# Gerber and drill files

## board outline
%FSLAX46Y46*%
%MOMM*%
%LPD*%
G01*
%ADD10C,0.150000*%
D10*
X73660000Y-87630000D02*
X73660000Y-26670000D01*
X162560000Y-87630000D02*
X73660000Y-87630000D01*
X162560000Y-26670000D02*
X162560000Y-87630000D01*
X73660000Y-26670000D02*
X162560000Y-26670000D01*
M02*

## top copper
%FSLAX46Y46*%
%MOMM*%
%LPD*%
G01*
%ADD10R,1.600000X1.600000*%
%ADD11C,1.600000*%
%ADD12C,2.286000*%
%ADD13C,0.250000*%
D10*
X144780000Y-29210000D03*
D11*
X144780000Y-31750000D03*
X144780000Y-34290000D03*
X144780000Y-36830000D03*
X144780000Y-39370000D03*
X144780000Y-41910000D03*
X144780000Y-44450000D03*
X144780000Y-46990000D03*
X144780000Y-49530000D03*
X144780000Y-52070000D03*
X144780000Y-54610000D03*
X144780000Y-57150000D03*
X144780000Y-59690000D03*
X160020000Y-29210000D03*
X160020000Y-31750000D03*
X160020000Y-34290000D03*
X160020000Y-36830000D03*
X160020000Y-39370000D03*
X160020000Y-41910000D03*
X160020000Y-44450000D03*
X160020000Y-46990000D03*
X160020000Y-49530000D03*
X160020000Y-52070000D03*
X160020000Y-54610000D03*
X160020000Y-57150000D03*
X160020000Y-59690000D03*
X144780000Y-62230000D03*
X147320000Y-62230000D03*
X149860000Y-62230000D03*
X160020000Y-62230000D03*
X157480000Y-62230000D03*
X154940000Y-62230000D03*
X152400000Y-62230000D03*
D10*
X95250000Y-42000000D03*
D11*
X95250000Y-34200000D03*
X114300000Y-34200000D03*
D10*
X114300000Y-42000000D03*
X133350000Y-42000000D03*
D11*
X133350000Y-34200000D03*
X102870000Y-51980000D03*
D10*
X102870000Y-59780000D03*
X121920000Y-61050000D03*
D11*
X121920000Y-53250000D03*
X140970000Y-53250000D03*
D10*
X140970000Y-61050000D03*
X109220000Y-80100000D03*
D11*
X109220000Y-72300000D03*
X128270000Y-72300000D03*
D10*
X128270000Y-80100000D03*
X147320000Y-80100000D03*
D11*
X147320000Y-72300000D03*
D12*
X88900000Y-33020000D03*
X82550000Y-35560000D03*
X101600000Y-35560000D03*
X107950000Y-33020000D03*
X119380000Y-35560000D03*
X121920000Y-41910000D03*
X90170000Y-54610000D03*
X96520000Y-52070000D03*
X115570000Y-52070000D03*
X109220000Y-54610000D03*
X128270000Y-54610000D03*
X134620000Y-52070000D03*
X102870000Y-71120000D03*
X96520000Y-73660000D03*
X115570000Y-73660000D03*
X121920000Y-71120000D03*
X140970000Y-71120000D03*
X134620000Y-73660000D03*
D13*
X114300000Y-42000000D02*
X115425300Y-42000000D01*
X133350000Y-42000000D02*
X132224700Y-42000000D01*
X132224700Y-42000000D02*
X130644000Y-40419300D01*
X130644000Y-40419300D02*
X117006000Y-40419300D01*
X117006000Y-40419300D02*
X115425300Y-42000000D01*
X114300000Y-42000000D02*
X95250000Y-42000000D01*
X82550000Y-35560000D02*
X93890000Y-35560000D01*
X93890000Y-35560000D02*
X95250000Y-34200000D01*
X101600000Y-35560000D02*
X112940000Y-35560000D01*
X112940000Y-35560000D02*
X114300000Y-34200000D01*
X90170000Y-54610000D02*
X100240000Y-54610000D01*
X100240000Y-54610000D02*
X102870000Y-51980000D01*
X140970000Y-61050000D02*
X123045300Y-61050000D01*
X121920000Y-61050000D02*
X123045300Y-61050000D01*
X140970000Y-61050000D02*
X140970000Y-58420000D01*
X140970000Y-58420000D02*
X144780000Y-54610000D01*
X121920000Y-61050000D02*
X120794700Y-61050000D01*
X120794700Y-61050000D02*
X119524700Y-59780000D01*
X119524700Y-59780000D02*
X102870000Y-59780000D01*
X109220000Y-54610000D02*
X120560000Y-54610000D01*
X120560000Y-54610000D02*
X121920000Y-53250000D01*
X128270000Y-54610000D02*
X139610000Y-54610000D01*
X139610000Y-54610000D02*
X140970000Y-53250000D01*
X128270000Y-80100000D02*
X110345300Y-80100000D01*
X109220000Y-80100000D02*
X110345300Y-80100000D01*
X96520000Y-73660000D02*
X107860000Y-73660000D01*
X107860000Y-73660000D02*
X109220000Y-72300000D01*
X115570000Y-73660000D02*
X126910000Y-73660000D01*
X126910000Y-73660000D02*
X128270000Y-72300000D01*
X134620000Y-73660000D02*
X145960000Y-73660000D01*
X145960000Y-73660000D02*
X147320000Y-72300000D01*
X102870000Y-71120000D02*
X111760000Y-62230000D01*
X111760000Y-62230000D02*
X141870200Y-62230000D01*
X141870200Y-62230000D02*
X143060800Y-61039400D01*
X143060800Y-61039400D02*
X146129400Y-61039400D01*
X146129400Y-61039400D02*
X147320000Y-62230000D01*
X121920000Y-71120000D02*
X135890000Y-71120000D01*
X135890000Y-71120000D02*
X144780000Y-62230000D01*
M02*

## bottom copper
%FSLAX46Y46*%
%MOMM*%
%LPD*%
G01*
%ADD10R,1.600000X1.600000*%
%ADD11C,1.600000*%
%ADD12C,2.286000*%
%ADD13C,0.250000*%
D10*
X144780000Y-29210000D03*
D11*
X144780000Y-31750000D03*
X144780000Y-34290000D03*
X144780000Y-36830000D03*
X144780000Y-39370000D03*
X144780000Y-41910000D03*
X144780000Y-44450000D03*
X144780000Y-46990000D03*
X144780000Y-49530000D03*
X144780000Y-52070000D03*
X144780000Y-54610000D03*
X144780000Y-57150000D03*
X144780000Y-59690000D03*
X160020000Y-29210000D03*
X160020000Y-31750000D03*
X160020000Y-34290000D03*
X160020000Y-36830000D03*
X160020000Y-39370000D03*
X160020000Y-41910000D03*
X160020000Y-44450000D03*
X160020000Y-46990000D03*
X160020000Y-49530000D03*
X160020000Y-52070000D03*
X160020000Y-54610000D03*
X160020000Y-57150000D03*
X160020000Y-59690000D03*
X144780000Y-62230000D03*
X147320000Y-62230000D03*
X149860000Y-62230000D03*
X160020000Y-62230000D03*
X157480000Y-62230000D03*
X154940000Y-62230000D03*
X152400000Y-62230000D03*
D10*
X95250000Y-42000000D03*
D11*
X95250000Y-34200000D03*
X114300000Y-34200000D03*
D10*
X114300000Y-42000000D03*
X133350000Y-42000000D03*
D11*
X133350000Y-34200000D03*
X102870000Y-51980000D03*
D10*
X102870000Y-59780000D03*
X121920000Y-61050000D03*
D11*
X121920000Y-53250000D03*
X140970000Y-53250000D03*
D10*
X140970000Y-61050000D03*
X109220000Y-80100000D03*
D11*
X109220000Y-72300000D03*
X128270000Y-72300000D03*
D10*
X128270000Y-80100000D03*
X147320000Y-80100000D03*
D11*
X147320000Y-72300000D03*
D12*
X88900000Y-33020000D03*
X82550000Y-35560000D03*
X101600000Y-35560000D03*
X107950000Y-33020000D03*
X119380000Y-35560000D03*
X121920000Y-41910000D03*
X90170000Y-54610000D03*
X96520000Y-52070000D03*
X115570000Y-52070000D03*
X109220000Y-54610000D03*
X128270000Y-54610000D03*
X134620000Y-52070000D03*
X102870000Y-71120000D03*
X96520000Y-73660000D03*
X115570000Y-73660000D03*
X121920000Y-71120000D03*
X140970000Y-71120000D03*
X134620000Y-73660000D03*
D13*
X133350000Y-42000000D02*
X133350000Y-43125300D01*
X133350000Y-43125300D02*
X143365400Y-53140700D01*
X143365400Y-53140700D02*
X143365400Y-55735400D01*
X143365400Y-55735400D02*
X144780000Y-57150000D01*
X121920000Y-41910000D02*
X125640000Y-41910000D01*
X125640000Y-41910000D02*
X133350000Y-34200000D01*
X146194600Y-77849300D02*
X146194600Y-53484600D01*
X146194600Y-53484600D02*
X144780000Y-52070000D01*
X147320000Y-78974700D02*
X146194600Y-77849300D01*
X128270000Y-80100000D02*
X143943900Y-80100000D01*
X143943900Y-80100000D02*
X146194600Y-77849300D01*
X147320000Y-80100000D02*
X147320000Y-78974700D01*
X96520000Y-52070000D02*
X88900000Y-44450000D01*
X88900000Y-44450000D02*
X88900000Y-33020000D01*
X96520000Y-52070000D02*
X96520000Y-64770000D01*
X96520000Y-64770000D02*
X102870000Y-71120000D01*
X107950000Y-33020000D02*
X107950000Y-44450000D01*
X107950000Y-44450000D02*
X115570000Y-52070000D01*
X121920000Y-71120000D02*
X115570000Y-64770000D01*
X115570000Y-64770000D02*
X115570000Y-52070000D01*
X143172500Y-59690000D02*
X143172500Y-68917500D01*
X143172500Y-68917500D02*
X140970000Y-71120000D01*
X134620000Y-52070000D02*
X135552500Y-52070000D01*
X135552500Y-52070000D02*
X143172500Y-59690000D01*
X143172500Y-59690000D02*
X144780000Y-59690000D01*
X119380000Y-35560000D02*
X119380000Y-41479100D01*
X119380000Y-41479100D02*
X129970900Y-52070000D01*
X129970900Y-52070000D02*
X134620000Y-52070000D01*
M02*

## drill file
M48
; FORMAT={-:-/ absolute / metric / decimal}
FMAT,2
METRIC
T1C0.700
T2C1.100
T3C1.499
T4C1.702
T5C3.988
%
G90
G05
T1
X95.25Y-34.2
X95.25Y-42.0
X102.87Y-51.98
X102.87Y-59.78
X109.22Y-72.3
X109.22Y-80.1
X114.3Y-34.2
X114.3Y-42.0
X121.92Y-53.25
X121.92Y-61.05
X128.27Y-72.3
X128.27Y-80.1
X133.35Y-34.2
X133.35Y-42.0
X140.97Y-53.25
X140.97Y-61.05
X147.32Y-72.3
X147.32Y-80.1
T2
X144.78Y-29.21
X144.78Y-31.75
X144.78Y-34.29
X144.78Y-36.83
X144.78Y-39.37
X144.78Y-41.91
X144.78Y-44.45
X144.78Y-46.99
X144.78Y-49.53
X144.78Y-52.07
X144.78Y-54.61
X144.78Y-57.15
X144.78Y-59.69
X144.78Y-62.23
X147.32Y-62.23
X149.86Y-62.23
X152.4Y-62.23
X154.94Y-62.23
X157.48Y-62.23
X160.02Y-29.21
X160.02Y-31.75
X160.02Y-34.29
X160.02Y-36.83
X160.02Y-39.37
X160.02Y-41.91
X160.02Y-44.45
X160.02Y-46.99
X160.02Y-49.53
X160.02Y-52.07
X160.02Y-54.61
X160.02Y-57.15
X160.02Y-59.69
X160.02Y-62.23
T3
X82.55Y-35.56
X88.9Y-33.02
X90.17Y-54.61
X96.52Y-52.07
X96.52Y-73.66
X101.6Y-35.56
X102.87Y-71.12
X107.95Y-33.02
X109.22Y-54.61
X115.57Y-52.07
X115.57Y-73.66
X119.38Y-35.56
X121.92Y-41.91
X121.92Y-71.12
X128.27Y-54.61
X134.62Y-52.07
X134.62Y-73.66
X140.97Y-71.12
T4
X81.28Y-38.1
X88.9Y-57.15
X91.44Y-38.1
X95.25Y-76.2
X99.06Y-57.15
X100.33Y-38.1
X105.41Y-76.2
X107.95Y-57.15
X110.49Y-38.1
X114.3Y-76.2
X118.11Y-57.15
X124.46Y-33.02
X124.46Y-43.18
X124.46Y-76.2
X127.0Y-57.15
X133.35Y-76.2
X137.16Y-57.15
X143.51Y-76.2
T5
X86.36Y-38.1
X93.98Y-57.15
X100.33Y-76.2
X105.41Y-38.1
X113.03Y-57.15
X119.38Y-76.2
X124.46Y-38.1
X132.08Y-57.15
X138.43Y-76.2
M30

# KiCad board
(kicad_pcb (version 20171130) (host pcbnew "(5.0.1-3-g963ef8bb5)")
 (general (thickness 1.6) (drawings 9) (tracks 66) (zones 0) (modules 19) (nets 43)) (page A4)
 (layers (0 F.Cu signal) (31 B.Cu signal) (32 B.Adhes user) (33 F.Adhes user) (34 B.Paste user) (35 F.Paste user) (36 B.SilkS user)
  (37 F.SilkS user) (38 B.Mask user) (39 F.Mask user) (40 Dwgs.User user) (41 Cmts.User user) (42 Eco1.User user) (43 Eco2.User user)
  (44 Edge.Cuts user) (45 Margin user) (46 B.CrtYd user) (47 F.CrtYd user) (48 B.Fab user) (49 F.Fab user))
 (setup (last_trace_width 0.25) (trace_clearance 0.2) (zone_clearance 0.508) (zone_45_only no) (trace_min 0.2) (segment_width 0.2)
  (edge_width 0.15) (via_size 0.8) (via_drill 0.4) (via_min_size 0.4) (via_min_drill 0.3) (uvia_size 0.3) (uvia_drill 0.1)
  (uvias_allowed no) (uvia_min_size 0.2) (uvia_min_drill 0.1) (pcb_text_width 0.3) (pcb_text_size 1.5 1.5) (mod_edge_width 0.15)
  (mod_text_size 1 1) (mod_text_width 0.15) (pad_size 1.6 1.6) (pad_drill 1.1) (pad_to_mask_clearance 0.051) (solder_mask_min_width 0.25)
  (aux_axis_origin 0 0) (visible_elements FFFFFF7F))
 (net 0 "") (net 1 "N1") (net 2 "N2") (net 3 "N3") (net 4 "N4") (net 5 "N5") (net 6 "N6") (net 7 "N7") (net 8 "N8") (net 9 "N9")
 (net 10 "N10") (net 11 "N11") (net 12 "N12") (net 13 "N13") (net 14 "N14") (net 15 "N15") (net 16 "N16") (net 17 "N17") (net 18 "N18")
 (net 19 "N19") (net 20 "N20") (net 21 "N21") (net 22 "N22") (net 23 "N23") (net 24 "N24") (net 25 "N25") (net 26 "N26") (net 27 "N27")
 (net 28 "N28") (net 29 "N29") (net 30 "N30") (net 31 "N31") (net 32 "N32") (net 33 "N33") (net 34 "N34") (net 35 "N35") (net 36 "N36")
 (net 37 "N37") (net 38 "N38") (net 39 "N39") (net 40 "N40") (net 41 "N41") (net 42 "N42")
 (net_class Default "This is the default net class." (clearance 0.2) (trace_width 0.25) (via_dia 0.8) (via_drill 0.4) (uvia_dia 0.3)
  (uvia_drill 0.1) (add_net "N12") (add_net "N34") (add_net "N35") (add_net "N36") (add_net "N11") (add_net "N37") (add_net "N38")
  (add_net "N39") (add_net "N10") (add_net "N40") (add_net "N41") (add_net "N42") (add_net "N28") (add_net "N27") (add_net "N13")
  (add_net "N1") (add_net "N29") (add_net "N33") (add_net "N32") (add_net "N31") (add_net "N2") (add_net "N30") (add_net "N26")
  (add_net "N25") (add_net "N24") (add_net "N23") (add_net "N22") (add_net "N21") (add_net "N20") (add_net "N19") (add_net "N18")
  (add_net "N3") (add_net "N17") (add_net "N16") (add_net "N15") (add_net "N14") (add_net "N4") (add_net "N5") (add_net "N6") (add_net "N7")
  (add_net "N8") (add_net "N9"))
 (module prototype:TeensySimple (layer F.Cu) (at 152.4 45.72 270)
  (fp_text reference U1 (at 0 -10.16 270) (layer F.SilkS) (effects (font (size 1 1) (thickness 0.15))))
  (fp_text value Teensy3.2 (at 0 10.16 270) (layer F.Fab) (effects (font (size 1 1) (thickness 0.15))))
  (pad 1 thru_hole rect (at -16.51 7.62 270) (size 1.6 1.6) (drill 1.1) (layers *.Cu *.Mask F.SilkS) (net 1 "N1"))
  (pad 2 thru_hole circle (at -13.97 7.62 270) (size 1.6 1.6) (drill 1.1) (layers *.Cu *.Mask F.SilkS) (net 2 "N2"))
  (pad 3 thru_hole circle (at -11.43 7.62 270) (size 1.6 1.6) (drill 1.1) (layers *.Cu *.Mask F.SilkS) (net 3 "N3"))
  (pad 4 thru_hole circle (at -8.89 7.62 270) (size 1.6 1.6) (drill 1.1) (layers *.Cu *.Mask F.SilkS) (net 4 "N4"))
  (pad 5 thru_hole circle (at -6.35 7.62 270) (size 1.6 1.6) (drill 1.1) (layers *.Cu *.Mask F.SilkS) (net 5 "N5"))
  (pad 6 thru_hole circle (at -3.81 7.62 270) (size 1.6 1.6) (drill 1.1) (layers *.Cu *.Mask F.SilkS) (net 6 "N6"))
  (pad 7 thru_hole circle (at -1.27 7.62 270) (size 1.6 1.6) (drill 1.1) (layers *.Cu *.Mask F.SilkS) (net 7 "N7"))
  (pad 8 thru_hole circle (at 1.27 7.62 270) (size 1.6 1.6) (drill 1.1) (layers *.Cu *.Mask F.SilkS) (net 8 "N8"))
  (pad 9 thru_hole circle (at 3.81 7.62 270) (size 1.6 1.6) (drill 1.1) (layers *.Cu *.Mask F.SilkS) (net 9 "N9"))
  (pad 10 thru_hole circle (at 6.35 7.62 270) (size 1.6 1.6) (drill 1.1) (layers *.Cu *.Mask F.SilkS) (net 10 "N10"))
  (pad 11 thru_hole circle (at 8.89 7.62 270) (size 1.6 1.6) (drill 1.1) (layers *.Cu *.Mask F.SilkS) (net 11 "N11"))
  (pad 12 thru_hole circle (at 11.43 7.62 270) (size 1.6 1.6) (drill 1.1) (layers *.Cu *.Mask F.SilkS) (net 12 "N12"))
  (pad 13 thru_hole circle (at 13.97 7.62 270) (size 1.6 1.6) (drill 1.1) (layers *.Cu *.Mask F.SilkS) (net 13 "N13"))
  (pad 33 thru_hole circle (at -16.51 -7.62 270) (size 1.6 1.6) (drill 1.1) (layers *.Cu *.Mask F.SilkS) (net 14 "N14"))
  (pad 32 thru_hole circle (at -13.97 -7.62 270) (size 1.6 1.6) (drill 1.1) (layers *.Cu *.Mask F.SilkS) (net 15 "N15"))
  (pad 31 thru_hole circle (at -11.43 -7.62 270) (size 1.6 1.6) (drill 1.1) (layers *.Cu *.Mask F.SilkS) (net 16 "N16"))
  (pad 30 thru_hole circle (at -8.89 -7.62 270) (size 1.6 1.6) (drill 1.1) (layers *.Cu *.Mask F.SilkS) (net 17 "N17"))
  (pad 29 thru_hole circle (at -6.35 -7.62 270) (size 1.6 1.6) (drill 1.1) (layers *.Cu *.Mask F.SilkS) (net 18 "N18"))
  (pad 28 thru_hole circle (at -3.81 -7.62 270) (size 1.6 1.6) (drill 1.1) (layers *.Cu *.Mask F.SilkS) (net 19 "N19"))
  (pad 27 thru_hole circle (at -1.27 -7.62 270) (size 1.6 1.6) (drill 1.1) (layers *.Cu *.Mask F.SilkS) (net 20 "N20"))
  (pad 26 thru_hole circle (at 1.27 -7.62 270) (size 1.6 1.6) (drill 1.1) (layers *.Cu *.Mask F.SilkS) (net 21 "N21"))
  (pad 25 thru_hole circle (at 3.81 -7.62 270) (size 1.6 1.6) (drill 1.1) (layers *.Cu *.Mask F.SilkS) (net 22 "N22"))
  (pad 24 thru_hole circle (at 6.35 -7.62 270) (size 1.6 1.6) (drill 1.1) (layers *.Cu *.Mask F.SilkS) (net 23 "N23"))
  (pad 23 thru_hole circle (at 8.89 -7.62 270) (size 1.6 1.6) (drill 1.1) (layers *.Cu *.Mask F.SilkS) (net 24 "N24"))
  (pad 22 thru_hole circle (at 11.43 -7.62 270) (size 1.6 1.6) (drill 1.1) (layers *.Cu *.Mask F.SilkS) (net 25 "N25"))
  (pad 21 thru_hole circle (at 13.97 -7.62 270) (size 1.6 1.6) (drill 1.1) (layers *.Cu *.Mask F.SilkS) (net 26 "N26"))
  (pad 14 thru_hole circle (at 16.51 7.62 270) (size 1.6 1.6) (drill 1.1) (layers *.Cu *.Mask F.SilkS) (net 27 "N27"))
  (pad 15 thru_hole circle (at 16.51 5.08 270) (size 1.6 1.6) (drill 1.1) (layers *.Cu *.Mask F.SilkS) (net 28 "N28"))
  (pad 16 thru_hole circle (at 16.51 2.54 270) (size 1.6 1.6) (drill 1.1) (layers *.Cu *.Mask F.SilkS) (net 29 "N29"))
  (pad 20 thru_hole circle (at 16.51 -7.62 270) (size 1.6 1.6) (drill 1.1) (layers *.Cu *.Mask F.SilkS) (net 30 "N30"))
  (pad 19 thru_hole circle (at 16.51 -5.08 270) (size 1.6 1.6) (drill 1.1) (layers *.Cu *.Mask F.SilkS) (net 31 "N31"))
  (pad 18 thru_hole circle (at 16.51 -2.54 270) (size 1.6 1.6) (drill 1.1) (layers *.Cu *.Mask F.SilkS) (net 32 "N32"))
  (pad 17 thru_hole circle (at 16.51 0 270) (size 1.6 1.6) (drill 1.1) (layers *.Cu *.Mask F.SilkS) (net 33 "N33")))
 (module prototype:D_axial (layer F.Cu) (at 95.25 38.1 90)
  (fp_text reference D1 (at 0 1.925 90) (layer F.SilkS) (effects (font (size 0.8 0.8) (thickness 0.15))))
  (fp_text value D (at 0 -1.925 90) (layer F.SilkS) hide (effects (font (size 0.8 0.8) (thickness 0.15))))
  (pad 1 thru_hole rect (at -3.9 0 90) (size 1.6 1.6) (drill 0.7) (layers *.Cu *.Mask F.SilkS) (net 12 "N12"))
  (pad 2 thru_hole circle (at 3.9 0 90) (size 1.6 1.6) (drill 0.7) (layers *.Cu *.Mask F.SilkS) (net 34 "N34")))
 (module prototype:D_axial (layer F.Cu) (at 114.3 38.1 90)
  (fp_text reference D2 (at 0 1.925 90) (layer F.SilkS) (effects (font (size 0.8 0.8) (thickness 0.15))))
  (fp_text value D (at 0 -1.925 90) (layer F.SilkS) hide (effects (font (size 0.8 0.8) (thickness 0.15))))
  (pad 2 thru_hole circle (at 3.9 0 90) (size 1.6 1.6) (drill 0.7) (layers *.Cu *.Mask F.SilkS) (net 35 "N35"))
  (pad 1 thru_hole rect (at -3.9 0 90) (size 1.6 1.6) (drill 0.7) (layers *.Cu *.Mask F.SilkS) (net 12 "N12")))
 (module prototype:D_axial (layer F.Cu) (at 133.35 38.1 90)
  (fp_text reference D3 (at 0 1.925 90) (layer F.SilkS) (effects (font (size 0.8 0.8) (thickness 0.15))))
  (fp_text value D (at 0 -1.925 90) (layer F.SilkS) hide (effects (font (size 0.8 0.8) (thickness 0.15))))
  (pad 1 thru_hole rect (at -3.9 0 90) (size 1.6 1.6) (drill 0.7) (layers *.Cu *.Mask F.SilkS) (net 12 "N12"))
  (pad 2 thru_hole circle (at 3.9 0 90) (size 1.6 1.6) (drill 0.7) (layers *.Cu *.Mask F.SilkS) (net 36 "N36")))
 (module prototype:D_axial (layer F.Cu) (at 102.87 55.88 90)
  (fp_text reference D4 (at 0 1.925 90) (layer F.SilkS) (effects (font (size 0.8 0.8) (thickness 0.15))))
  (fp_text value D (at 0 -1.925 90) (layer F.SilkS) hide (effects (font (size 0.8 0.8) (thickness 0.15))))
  (pad 2 thru_hole circle (at 3.9 0 90) (size 1.6 1.6) (drill 0.7) (layers *.Cu *.Mask F.SilkS) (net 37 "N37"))
  (pad 1 thru_hole rect (at -3.9 0 90) (size 1.6 1.6) (drill 0.7) (layers *.Cu *.Mask F.SilkS) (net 11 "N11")))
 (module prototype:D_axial (layer F.Cu) (at 121.92 57.15 90)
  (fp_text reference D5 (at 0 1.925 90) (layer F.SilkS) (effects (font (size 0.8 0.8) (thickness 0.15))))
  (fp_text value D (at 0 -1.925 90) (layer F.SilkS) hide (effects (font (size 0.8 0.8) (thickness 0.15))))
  (pad 1 thru_hole rect (at -3.9 0 90) (size 1.6 1.6) (drill 0.7) (layers *.Cu *.Mask F.SilkS) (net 11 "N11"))
  (pad 2 thru_hole circle (at 3.9 0 90) (size 1.6 1.6) (drill 0.7) (layers *.Cu *.Mask F.SilkS) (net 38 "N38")))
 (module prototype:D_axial (layer F.Cu) (at 140.97 57.15 90)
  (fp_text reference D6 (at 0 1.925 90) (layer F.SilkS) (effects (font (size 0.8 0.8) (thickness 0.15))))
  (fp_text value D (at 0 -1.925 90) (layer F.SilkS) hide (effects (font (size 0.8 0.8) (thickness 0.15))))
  (pad 2 thru_hole circle (at 3.9 0 90) (size 1.6 1.6) (drill 0.7) (layers *.Cu *.Mask F.SilkS) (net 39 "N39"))
  (pad 1 thru_hole rect (at -3.9 0 90) (size 1.6 1.6) (drill 0.7) (layers *.Cu *.Mask F.SilkS) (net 11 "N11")))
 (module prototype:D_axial (layer F.Cu) (at 109.22 76.2 90)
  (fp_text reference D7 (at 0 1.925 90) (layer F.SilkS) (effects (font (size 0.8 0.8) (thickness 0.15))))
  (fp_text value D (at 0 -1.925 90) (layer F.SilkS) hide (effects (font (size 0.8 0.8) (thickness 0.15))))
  (pad 1 thru_hole rect (at -3.9 0 90) (size 1.6 1.6) (drill 0.7) (layers *.Cu *.Mask F.SilkS) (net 10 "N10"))
  (pad 2 thru_hole circle (at 3.9 0 90) (size 1.6 1.6) (drill 0.7) (layers *.Cu *.Mask F.SilkS) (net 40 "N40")))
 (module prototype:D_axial (layer F.Cu) (at 128.27 76.2 90)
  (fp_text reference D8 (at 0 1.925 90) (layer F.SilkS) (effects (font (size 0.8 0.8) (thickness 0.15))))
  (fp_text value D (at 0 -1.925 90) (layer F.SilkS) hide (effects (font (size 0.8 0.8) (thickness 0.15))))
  (pad 2 thru_hole circle (at 3.9 0 90) (size 1.6 1.6) (drill 0.7) (layers *.Cu *.Mask F.SilkS) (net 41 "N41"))
  (pad 1 thru_hole rect (at -3.9 0 90) (size 1.6 1.6) (drill 0.7) (layers *.Cu *.Mask F.SilkS) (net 10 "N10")))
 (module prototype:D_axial (layer F.Cu) (at 147.32 76.2 90)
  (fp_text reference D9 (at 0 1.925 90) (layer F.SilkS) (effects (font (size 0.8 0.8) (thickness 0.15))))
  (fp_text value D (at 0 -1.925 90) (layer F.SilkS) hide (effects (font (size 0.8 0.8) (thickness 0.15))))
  (pad 1 thru_hole rect (at -3.9 0 90) (size 1.6 1.6) (drill 0.7) (layers *.Cu *.Mask F.SilkS) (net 10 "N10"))
  (pad 2 thru_hole circle (at 3.9 0 90) (size 1.6 1.6) (drill 0.7) (layers *.Cu *.Mask F.SilkS) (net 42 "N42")))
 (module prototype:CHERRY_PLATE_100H (layer F.Cu) (at 86.36 38.1)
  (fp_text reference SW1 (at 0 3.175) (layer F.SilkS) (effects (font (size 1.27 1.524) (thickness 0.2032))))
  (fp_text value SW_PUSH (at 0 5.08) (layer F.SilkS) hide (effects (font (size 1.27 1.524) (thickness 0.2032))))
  (pad 1 thru_hole circle (at 2.54 -5.08) (size 2.286 2.286) (drill 1.4986) (layers *.Cu *.SilkS *.Mask) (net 28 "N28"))
  (pad 2 thru_hole circle (at -3.81 -2.54) (size 2.286 2.286) (drill 1.4986) (layers *.Cu *.SilkS *.Mask) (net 34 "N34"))
  (pad HOLE np_thru_hole circle (at 0 0) (size 3.9878 3.9878) (drill 3.9878) (layers *.Cu))
  (pad HOLE np_thru_hole circle (at -5.08 0) (size 1.7018 1.7018) (drill 1.7018) (layers *.Cu))
  (pad HOLE np_thru_hole circle (at 5.08 0) (size 1.7018 1.7018) (drill 1.7018) (layers *.Cu)))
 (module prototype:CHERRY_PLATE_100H (layer F.Cu) (at 105.41 38.1)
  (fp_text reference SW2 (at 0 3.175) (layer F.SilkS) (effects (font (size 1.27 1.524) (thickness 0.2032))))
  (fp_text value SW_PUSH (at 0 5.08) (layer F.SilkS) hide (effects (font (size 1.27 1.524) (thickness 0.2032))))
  (pad HOLE np_thru_hole circle (at 5.08 0) (size 1.7018 1.7018) (drill 1.7018) (layers *.Cu))
  (pad HOLE np_thru_hole circle (at -5.08 0) (size 1.7018 1.7018) (drill 1.7018) (layers *.Cu))
  (pad HOLE np_thru_hole circle (at 0 0) (size 3.9878 3.9878) (drill 3.9878) (layers *.Cu))
  (pad 2 thru_hole circle (at -3.81 -2.54) (size 2.286 2.286) (drill 1.4986) (layers *.Cu *.SilkS *.Mask) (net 35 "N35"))
  (pad 1 thru_hole circle (at 2.54 -5.08) (size 2.286 2.286) (drill 1.4986) (layers *.Cu *.SilkS *.Mask) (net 27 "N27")))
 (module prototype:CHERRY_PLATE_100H (layer F.Cu) (at 124.46 38.1 90)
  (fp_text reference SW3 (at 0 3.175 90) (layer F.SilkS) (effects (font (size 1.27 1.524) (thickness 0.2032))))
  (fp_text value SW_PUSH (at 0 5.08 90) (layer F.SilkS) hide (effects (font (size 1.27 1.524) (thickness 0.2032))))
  (pad 1 thru_hole circle (at 2.54 -5.08 90) (size 2.286 2.286) (drill 1.4986) (layers *.Cu *.SilkS *.Mask) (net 13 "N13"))
  (pad 2 thru_hole circle (at -3.81 -2.54 90) (size 2.286 2.286) (drill 1.4986) (layers *.Cu *.SilkS *.Mask) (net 36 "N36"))
  (pad HOLE np_thru_hole circle (at 0 0 90) (size 3.9878 3.9878) (drill 3.9878) (layers *.Cu))
  (pad HOLE np_thru_hole circle (at -5.08 0 90) (size 1.7018 1.7018) (drill 1.7018) (layers *.Cu))
  (pad HOLE np_thru_hole circle (at 5.08 0 90) (size 1.7018 1.7018) (drill 1.7018) (layers *.Cu)))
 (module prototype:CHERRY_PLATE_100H (layer F.Cu) (at 93.98 57.15)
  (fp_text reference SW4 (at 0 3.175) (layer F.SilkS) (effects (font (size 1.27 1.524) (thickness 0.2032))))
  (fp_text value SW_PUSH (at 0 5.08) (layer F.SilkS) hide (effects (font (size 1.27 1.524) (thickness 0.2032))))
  (pad HOLE np_thru_hole circle (at 5.08 0) (size 1.7018 1.7018) (drill 1.7018) (layers *.Cu))
  (pad HOLE np_thru_hole circle (at -5.08 0) (size 1.7018 1.7018) (drill 1.7018) (layers *.Cu))
  (pad HOLE np_thru_hole circle (at 0 0) (size 3.9878 3.9878) (drill 3.9878) (layers *.Cu))
  (pad 2 thru_hole circle (at -3.81 -2.54) (size 2.286 2.286) (drill 1.4986) (layers *.Cu *.SilkS *.Mask) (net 37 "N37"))
  (pad 1 thru_hole circle (at 2.54 -5.08) (size 2.286 2.286) (drill 1.4986) (layers *.Cu *.SilkS *.Mask) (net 28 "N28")))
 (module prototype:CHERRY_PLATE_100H (layer F.Cu) (at 113.03 57.15)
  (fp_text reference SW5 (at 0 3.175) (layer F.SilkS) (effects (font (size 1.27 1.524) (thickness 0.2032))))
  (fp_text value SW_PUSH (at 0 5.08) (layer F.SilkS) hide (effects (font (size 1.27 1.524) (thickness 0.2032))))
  (pad 1 thru_hole circle (at 2.54 -5.08) (size 2.286 2.286) (drill 1.4986) (layers *.Cu *.SilkS *.Mask) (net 27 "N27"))
  (pad 2 thru_hole circle (at -3.81 -2.54) (size 2.286 2.286) (drill 1.4986) (layers *.Cu *.SilkS *.Mask) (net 38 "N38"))
  (pad HOLE np_thru_hole circle (at 0 0) (size 3.9878 3.9878) (drill 3.9878) (layers *.Cu))
  (pad HOLE np_thru_hole circle (at -5.08 0) (size 1.7018 1.7018) (drill 1.7018) (layers *.Cu))
  (pad HOLE np_thru_hole circle (at 5.08 0) (size 1.7018 1.7018) (drill 1.7018) (layers *.Cu)))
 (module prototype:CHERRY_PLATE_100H (layer F.Cu) (at 132.08 57.15)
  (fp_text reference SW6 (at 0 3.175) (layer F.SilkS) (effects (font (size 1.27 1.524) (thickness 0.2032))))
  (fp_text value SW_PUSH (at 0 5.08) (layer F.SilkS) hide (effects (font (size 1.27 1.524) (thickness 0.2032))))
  (pad HOLE np_thru_hole circle (at 5.08 0) (size 1.7018 1.7018) (drill 1.7018) (layers *.Cu))
  (pad HOLE np_thru_hole circle (at -5.08 0) (size 1.7018 1.7018) (drill 1.7018) (layers *.Cu))
  (pad HOLE np_thru_hole circle (at 0 0) (size 3.9878 3.9878) (drill 3.9878) (layers *.Cu))
  (pad 2 thru_hole circle (at -3.81 -2.54) (size 2.286 2.286) (drill 1.4986) (layers *.Cu *.SilkS *.Mask) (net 39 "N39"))
  (pad 1 thru_hole circle (at 2.54 -5.08) (size 2.286 2.286) (drill 1.4986) (layers *.Cu *.SilkS *.Mask) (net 13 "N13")))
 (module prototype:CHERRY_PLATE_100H (layer F.Cu) (at 100.33 76.2)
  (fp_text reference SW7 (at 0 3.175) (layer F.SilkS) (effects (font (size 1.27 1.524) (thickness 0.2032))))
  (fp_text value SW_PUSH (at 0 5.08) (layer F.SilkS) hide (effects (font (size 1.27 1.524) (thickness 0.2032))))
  (pad 1 thru_hole circle (at 2.54 -5.08) (size 2.286 2.286) (drill 1.4986) (layers *.Cu *.SilkS *.Mask) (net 28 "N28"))
  (pad 2 thru_hole circle (at -3.81 -2.54) (size 2.286 2.286) (drill 1.4986) (layers *.Cu *.SilkS *.Mask) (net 40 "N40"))
  (pad HOLE np_thru_hole circle (at 0 0) (size 3.9878 3.9878) (drill 3.9878) (layers *.Cu))
  (pad HOLE np_thru_hole circle (at -5.08 0) (size 1.7018 1.7018) (drill 1.7018) (layers *.Cu))
  (pad HOLE np_thru_hole circle (at 5.08 0) (size 1.7018 1.7018) (drill 1.7018) (layers *.Cu)))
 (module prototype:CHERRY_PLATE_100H (layer F.Cu) (at 119.38 76.2)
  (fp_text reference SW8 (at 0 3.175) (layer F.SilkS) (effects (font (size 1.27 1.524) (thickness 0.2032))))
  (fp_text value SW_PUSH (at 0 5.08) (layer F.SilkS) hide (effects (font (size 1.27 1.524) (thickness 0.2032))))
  (pad HOLE np_thru_hole circle (at 5.08 0) (size 1.7018 1.7018) (drill 1.7018) (layers *.Cu))
  (pad HOLE np_thru_hole circle (at -5.08 0) (size 1.7018 1.7018) (drill 1.7018) (layers *.Cu))
  (pad HOLE np_thru_hole circle (at 0 0) (size 3.9878 3.9878) (drill 3.9878) (layers *.Cu))
  (pad 2 thru_hole circle (at -3.81 -2.54) (size 2.286 2.286) (drill 1.4986) (layers *.Cu *.SilkS *.Mask) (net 41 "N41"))
  (pad 1 thru_hole circle (at 2.54 -5.08) (size 2.286 2.286) (drill 1.4986) (layers *.Cu *.SilkS *.Mask) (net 27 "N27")))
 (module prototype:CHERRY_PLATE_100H (layer F.Cu) (at 138.43 76.2)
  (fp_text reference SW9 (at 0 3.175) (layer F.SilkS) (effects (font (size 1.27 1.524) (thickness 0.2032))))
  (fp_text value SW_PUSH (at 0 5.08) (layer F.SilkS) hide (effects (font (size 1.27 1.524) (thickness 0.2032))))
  (pad 1 thru_hole circle (at 2.54 -5.08) (size 2.286 2.286) (drill 1.4986) (layers *.Cu *.SilkS *.Mask) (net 13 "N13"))
  (pad 2 thru_hole circle (at -3.81 -2.54) (size 2.286 2.286) (drill 1.4986) (layers *.Cu *.SilkS *.Mask) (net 42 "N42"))
  (pad HOLE np_thru_hole circle (at 0 0) (size 3.9878 3.9878) (drill 3.9878) (layers *.Cu))
  (pad HOLE np_thru_hole circle (at -5.08 0) (size 1.7018 1.7018) (drill 1.7018) (layers *.Cu))
  (pad HOLE np_thru_hole circle (at 5.08 0) (size 1.7018 1.7018) (drill 1.7018) (layers *.Cu)))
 (gr_line (start 73.66 87.63) (end 73.66 26.67) (layer Edge.Cuts) (width 0.15))
 (gr_line (start 162.56 87.63) (end 73.66 87.63) (layer Edge.Cuts) (width 0.15))
 (gr_line (start 162.56 26.67) (end 162.56 87.63) (layer Edge.Cuts) (width 0.15))
 (gr_line (start 73.66 26.67) (end 162.56 26.67) (layer Edge.Cuts) (width 0.15))
 (segment (start 133.35 42) (end 133.35 43.1253) (width 0.25) (layer B.Cu) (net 12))
 (segment (start 133.35 43.1253) (end 143.3654 53.1407) (width 0.25) (layer B.Cu) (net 12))
 (segment (start 143.3654 53.1407) (end 143.3654 55.7354) (width 0.25) (layer B.Cu) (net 12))
 (segment (start 143.3654 55.7354) (end 144.78 57.15) (width 0.25) (layer B.Cu) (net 12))
 (segment (start 114.3 42) (end 115.4253 42) (width 0.25) (layer F.Cu) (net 12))
 (segment (start 133.35 42) (end 132.2247 42) (width 0.25) (layer F.Cu) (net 12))
 (segment (start 132.2247 42) (end 130.644 40.4193) (width 0.25) (layer F.Cu) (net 12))
 (segment (start 130.644 40.4193) (end 117.006 40.4193) (width 0.25) (layer F.Cu) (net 12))
 (segment (start 117.006 40.4193) (end 115.4253 42) (width 0.25) (layer F.Cu) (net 12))
 (segment (start 114.3 42) (end 95.25 42) (width 0.25) (layer F.Cu) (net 12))
 (segment (start 82.55 35.56) (end 93.89 35.56) (width 0.25) (layer F.Cu) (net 34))
 (segment (start 93.89 35.56) (end 95.25 34.2) (width 0.25) (layer F.Cu) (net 34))
 (segment (start 101.6 35.56) (end 112.94 35.56) (width 0.25) (layer F.Cu) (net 35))
 (segment (start 112.94 35.56) (end 114.3 34.2) (width 0.25) (layer F.Cu) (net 35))
 (segment (start 121.92 41.91) (end 125.64 41.91) (width 0.25) (layer B.Cu) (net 36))
 (segment (start 125.64 41.91) (end 133.35 34.2) (width 0.25) (layer B.Cu) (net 36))
 (segment (start 90.17 54.61) (end 100.24 54.61) (width 0.25) (layer F.Cu) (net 37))
 (segment (start 100.24 54.61) (end 102.87 51.98) (width 0.25) (layer F.Cu) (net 37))
 (segment (start 140.97 61.05) (end 123.0453 61.05) (width 0.25) (layer F.Cu) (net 11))
 (segment (start 121.92 61.05) (end 123.0453 61.05) (width 0.25) (layer F.Cu) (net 11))
 (segment (start 140.97 61.05) (end 140.97 58.42) (width 0.25) (layer F.Cu) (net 11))
 (segment (start 140.97 58.42) (end 144.78 54.61) (width 0.25) (layer F.Cu) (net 11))
 (segment (start 121.92 61.05) (end 120.7947 61.05) (width 0.25) (layer F.Cu) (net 11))
 (segment (start 120.7947 61.05) (end 119.5247 59.78) (width 0.25) (layer F.Cu) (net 11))
 (segment (start 119.5247 59.78) (end 102.87 59.78) (width 0.25) (layer F.Cu) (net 11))
 (segment (start 109.22 54.61) (end 120.56 54.61) (width 0.25) (layer F.Cu) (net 38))
 (segment (start 120.56 54.61) (end 121.92 53.25) (width 0.25) (layer F.Cu) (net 38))
 (segment (start 128.27 54.61) (end 139.61 54.61) (width 0.25) (layer F.Cu) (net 39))
 (segment (start 139.61 54.61) (end 140.97 53.25) (width 0.25) (layer F.Cu) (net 39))
 (segment (start 146.1946 77.8493) (end 146.1946 53.4846) (width 0.25) (layer B.Cu) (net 10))
 (segment (start 146.1946 53.4846) (end 144.78 52.07) (width 0.25) (layer B.Cu) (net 10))
 (segment (start 147.32 78.9747) (end 146.1946 77.8493) (width 0.25) (layer B.Cu) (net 10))
 (segment (start 128.27 80.1) (end 143.9439 80.1) (width 0.25) (layer B.Cu) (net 10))
 (segment (start 143.9439 80.1) (end 146.1946 77.8493) (width 0.25) (layer B.Cu) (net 10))
 (segment (start 147.32 80.1) (end 147.32 78.9747) (width 0.25) (layer B.Cu) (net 10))
 (segment (start 128.27 80.1) (end 110.3453 80.1) (width 0.25) (layer F.Cu) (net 10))
 (segment (start 109.22 80.1) (end 110.3453 80.1) (width 0.25) (layer F.Cu) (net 10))
 (segment (start 96.52 73.66) (end 107.86 73.66) (width 0.25) (layer F.Cu) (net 40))
 (segment (start 107.86 73.66) (end 109.22 72.3) (width 0.25) (layer F.Cu) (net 40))
 (segment (start 115.57 73.66) (end 126.91 73.66) (width 0.25) (layer F.Cu) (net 41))
 (segment (start 126.91 73.66) (end 128.27 72.3) (width 0.25) (layer F.Cu) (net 41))
 (segment (start 134.62 73.66) (end 145.96 73.66) (width 0.25) (layer F.Cu) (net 42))
 (segment (start 145.96 73.66) (end 147.32 72.3) (width 0.25) (layer F.Cu) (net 42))
 (segment (start 102.87 71.12) (end 111.76 62.23) (width 0.25) (layer F.Cu) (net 28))
 (segment (start 111.76 62.23) (end 141.8702 62.23) (width 0.25) (layer F.Cu) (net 28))
 (segment (start 141.8702 62.23) (end 143.0608 61.0394) (width 0.25) (layer F.Cu) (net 28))
 (segment (start 143.0608 61.0394) (end 146.1294 61.0394) (width 0.25) (layer F.Cu) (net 28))
 (segment (start 146.1294 61.0394) (end 147.32 62.23) (width 0.25) (layer F.Cu) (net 28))
 (segment (start 96.52 52.07) (end 88.9 44.45) (width 0.25) (layer B.Cu) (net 28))
 (segment (start 88.9 44.45) (end 88.9 33.02) (width 0.25) (layer B.Cu) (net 28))
 (segment (start 96.52 52.07) (end 96.52 64.77) (width 0.25) (layer B.Cu) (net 28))
 (segment (start 96.52 64.77) (end 102.87 71.12) (width 0.25) (layer B.Cu) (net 28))
 (segment (start 121.92 71.12) (end 135.89 71.12) (width 0.25) (layer F.Cu) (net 27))
 (segment (start 135.89 71.12) (end 144.78 62.23) (width 0.25) (layer F.Cu) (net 27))
 (segment (start 107.95 33.02) (end 107.95 44.45) (width 0.25) (layer B.Cu) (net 27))
 (segment (start 107.95 44.45) (end 115.57 52.07) (width 0.25) (layer B.Cu) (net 27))
 (segment (start 121.92 71.12) (end 115.57 64.77) (width 0.25) (layer B.Cu) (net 27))
 (segment (start 115.57 64.77) (end 115.57 52.07) (width 0.25) (layer B.Cu) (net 27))
 (segment (start 143.1725 59.69) (end 143.1725 68.9175) (width 0.25) (layer B.Cu) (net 13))
 (segment (start 143.1725 68.9175) (end 140.97 71.12) (width 0.25) (layer B.Cu) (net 13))
 (segment (start 134.62 52.07) (end 135.5525 52.07) (width 0.25) (layer B.Cu) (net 13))
 (segment (start 135.5525 52.07) (end 143.1725 59.69) (width 0.25) (layer B.Cu) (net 13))
 (segment (start 143.1725 59.69) (end 144.78 59.69) (width 0.25) (layer B.Cu) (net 13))
 (segment (start 119.38 35.56) (end 119.38 41.4791) (width 0.25) (layer B.Cu) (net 13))
 (segment (start 119.38 41.4791) (end 129.9709 52.07) (width 0.25) (layer B.Cu) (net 13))
 (segment (start 129.9709 52.07) (end 134.62 52.07) (width 0.25) (layer B.Cu) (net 13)))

